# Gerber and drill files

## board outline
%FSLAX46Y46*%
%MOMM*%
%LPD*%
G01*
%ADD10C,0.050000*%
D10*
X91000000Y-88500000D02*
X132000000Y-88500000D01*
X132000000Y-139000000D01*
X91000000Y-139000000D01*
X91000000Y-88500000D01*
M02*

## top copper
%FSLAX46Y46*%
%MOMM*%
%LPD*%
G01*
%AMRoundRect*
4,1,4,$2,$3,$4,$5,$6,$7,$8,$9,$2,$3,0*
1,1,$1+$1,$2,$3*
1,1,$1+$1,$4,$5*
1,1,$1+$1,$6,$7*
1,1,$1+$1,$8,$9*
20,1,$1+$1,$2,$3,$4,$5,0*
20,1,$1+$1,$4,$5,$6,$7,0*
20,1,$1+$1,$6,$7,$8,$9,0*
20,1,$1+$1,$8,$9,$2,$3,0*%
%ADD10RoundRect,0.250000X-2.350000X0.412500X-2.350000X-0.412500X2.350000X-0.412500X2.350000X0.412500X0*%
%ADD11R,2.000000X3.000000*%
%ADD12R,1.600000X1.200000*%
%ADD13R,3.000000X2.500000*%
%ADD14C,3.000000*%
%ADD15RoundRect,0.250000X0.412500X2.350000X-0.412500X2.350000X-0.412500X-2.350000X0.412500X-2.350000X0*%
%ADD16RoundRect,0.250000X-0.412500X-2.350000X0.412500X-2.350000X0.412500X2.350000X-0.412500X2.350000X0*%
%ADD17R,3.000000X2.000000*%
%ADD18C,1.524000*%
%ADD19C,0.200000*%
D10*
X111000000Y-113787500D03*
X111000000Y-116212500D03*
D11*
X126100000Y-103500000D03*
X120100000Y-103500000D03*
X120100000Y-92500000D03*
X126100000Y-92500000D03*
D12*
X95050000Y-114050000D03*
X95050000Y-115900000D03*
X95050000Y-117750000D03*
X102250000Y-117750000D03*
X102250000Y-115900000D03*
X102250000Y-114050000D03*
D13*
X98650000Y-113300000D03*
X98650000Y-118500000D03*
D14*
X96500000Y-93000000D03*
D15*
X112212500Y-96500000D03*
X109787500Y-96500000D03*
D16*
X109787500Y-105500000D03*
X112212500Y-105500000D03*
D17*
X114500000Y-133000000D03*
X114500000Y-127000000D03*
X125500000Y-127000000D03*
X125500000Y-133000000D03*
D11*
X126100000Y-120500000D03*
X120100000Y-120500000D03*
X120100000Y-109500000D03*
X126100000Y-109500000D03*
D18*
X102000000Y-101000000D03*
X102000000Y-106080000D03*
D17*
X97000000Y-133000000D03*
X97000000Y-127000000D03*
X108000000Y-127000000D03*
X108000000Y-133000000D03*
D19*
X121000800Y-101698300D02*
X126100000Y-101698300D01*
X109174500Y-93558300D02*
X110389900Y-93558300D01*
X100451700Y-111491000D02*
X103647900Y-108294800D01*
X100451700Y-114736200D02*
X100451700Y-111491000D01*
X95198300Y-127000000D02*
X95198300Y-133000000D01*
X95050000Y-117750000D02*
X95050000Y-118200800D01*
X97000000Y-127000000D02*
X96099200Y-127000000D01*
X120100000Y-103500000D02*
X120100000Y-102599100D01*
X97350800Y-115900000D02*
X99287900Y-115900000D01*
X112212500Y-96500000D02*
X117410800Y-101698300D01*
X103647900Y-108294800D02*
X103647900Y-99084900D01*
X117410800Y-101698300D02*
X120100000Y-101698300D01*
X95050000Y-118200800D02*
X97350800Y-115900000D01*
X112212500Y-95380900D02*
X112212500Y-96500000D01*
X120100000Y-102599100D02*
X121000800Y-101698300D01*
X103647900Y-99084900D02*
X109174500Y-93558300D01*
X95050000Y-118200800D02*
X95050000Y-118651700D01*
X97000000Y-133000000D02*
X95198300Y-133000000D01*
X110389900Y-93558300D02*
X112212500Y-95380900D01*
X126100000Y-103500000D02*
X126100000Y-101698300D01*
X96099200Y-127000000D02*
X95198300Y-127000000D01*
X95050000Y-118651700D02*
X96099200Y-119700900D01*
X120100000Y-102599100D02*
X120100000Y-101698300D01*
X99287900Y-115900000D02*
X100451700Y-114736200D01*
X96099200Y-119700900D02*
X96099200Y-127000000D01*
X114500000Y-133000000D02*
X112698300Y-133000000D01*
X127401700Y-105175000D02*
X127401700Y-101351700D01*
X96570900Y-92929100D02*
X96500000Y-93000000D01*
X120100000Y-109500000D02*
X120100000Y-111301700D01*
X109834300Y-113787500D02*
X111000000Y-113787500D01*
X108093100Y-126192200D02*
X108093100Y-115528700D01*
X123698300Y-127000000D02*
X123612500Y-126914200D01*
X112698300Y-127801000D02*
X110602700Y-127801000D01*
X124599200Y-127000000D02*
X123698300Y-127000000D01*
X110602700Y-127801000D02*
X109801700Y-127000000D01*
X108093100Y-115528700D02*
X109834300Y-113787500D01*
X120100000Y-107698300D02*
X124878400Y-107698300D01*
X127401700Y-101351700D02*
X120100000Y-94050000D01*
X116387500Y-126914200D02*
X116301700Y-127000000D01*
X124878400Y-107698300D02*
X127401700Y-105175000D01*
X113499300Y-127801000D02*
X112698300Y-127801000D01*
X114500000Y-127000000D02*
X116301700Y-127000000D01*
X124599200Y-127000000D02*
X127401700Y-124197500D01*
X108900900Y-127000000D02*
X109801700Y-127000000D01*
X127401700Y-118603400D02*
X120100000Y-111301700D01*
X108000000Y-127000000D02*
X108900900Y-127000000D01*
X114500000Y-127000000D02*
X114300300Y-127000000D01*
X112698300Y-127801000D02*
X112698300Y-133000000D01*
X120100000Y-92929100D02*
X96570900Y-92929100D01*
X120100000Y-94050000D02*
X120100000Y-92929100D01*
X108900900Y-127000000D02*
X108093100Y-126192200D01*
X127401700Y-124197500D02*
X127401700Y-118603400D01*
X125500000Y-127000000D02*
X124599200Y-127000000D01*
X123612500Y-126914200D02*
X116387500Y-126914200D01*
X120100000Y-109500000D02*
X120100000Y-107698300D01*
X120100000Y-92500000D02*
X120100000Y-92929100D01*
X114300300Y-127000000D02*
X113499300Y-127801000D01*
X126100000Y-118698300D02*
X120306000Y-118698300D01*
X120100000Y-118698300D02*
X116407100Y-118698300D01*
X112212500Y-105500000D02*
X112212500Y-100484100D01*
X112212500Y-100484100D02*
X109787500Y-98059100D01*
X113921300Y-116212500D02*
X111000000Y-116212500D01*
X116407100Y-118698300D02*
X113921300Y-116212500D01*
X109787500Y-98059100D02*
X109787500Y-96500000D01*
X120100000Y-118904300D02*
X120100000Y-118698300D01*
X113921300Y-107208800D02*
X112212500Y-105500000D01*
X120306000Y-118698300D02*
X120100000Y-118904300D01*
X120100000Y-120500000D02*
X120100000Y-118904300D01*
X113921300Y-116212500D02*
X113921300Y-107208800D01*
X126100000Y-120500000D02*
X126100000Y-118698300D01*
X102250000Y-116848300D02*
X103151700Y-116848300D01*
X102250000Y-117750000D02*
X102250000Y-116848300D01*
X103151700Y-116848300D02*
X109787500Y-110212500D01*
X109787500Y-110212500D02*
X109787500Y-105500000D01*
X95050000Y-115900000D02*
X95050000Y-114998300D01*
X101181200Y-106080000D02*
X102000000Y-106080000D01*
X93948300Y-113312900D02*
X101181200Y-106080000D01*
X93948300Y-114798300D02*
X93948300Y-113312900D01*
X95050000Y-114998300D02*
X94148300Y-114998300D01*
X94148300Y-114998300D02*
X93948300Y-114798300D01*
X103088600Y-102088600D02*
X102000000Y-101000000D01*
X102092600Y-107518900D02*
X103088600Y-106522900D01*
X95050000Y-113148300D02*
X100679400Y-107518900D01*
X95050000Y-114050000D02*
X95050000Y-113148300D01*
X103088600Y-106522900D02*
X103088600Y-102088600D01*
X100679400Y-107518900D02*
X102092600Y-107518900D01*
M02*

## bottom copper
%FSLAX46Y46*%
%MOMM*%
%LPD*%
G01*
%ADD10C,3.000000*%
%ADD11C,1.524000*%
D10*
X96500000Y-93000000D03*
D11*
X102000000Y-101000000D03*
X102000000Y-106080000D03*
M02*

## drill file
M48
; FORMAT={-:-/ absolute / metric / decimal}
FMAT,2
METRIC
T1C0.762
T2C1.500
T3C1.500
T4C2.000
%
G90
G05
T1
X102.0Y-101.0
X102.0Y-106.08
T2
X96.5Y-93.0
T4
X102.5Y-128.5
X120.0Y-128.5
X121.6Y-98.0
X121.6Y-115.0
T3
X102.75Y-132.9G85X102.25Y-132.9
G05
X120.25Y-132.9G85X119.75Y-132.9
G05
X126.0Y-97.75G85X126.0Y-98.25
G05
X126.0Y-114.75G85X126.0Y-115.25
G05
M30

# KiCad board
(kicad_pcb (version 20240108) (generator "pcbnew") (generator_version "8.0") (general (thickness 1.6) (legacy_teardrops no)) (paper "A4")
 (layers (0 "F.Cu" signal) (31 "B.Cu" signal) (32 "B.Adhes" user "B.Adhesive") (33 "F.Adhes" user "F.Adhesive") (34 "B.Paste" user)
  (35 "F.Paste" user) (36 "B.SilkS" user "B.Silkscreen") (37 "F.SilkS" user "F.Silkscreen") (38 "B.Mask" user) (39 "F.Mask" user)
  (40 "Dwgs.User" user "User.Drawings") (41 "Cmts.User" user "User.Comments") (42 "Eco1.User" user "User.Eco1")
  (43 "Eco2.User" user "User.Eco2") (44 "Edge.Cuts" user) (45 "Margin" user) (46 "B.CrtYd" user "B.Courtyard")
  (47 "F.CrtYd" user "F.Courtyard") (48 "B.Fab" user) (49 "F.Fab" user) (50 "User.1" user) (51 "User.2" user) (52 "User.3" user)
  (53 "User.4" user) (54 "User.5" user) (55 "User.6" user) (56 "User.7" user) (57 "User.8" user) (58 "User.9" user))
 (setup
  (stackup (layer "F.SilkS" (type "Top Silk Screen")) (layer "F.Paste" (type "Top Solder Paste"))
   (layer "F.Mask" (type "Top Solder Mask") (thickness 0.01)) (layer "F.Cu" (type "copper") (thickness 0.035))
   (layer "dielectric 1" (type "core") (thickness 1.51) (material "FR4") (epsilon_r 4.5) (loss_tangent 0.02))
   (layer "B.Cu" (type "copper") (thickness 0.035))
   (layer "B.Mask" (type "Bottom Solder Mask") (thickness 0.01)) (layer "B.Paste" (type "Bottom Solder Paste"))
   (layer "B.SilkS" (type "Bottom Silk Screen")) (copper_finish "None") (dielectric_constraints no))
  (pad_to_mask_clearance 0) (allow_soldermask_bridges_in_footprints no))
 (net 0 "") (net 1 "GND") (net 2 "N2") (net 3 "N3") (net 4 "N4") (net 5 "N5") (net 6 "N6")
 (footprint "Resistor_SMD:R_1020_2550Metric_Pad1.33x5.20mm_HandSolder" (layer "F.Cu") (at 111 115 -90)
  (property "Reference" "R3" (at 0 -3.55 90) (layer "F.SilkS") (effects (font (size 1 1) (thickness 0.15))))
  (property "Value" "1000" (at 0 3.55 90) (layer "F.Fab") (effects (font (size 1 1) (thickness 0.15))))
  (pad "1" smd roundrect (at -1.2125 0 270) (size 1.325 5.2) (layers "F.Cu" "F.Paste" "F.Mask") (roundrect_rratio 0.188679) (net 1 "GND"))
  (pad "2" smd roundrect (at 1.2125 0 270) (size 1.325 5.2) (layers "F.Cu" "F.Paste" "F.Mask") (roundrect_rratio 0.188679) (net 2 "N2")))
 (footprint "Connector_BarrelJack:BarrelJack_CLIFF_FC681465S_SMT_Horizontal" (layer "F.Cu") (at 123.1 98 180)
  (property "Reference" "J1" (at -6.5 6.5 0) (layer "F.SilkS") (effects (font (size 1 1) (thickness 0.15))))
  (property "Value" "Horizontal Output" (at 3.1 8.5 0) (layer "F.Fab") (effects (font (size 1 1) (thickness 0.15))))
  (pad "" np_thru_hole oval (at -2.9 0 270) (size 2 1.5) (drill oval 2 1.5) (layers "*.Cu" "*.Mask"))
  (pad "" np_thru_hole circle (at 1.5 0 270) (size 2 2) (drill 2) (layers "*.Cu" "*.Mask"))
  (pad "1" smd rect (at -3 -5.5 270) (size 3 2) (layers "F.Cu" "F.Paste" "F.Mask") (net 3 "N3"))
  (pad "1" smd rect (at 3 -5.5 270) (size 3 2) (layers "F.Cu" "F.Paste" "F.Mask") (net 3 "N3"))
  (pad "2" smd rect (at 3 5.5 270) (size 3 2) (layers "F.Cu" "F.Paste" "F.Mask") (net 1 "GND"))
  (pad "3" smd rect (at -3 5.5 270) (size 3 2) (layers "F.Cu" "F.Paste" "F.Mask")))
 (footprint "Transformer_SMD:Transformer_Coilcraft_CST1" (layer "F.Cu") (at 98.65 115.9)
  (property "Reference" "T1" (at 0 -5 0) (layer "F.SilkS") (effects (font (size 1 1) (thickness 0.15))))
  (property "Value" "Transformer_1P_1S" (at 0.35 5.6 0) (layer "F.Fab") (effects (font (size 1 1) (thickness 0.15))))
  (pad "1" smd rect (at -3.6 -1.85) (size 1.6 1.2) (layers "F.Cu" "F.Paste" "F.Mask") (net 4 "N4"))
  (pad "2" smd rect (at -3.6 0) (size 1.6 1.2) (layers "F.Cu" "F.Paste" "F.Mask") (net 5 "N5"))
  (pad "3" smd rect (at -3.6 1.85) (size 1.6 1.2) (layers "F.Cu" "F.Paste" "F.Mask") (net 3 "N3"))
  (pad "4" smd rect (at 3.6 1.85) (size 1.6 1.2) (layers "F.Cu" "F.Paste" "F.Mask") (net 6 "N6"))
  (pad "5" smd rect (at 3.6 0) (size 1.6 1.2) (layers "F.Cu" "F.Paste" "F.Mask"))
  (pad "6" smd rect (at 3.6 -1.85) (size 1.6 1.2) (layers "F.Cu" "F.Paste" "F.Mask"))
  (pad "7" smd rect (at 0 -2.6) (size 3 2.5) (layers "F.Cu" "F.Paste" "F.Mask"))
  (pad "8" smd rect (at 0 2.6) (size 3 2.5) (layers "F.Cu" "F.Paste" "F.Mask")))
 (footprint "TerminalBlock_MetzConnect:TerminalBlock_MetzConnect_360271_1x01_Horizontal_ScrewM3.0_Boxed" (layer "F.Cu") (at 96.5 93)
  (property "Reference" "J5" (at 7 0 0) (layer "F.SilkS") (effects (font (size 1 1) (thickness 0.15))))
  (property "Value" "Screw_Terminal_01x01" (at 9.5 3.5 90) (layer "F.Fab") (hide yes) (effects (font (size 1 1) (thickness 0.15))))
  (pad "1" thru_hole circle (at 0 0) (size 3 3) (drill 1.5) (layers "*.Cu" "*.Mask") (remove_unused_layers no) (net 1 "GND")))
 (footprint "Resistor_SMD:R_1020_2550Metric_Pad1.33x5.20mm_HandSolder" (layer "F.Cu") (at 111 96.5 180)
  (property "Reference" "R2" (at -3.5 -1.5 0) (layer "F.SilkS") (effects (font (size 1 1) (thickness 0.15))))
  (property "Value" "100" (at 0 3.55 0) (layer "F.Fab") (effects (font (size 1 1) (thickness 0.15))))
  (pad "1" smd roundrect (at -1.2125 0 180) (size 1.325 5.2) (layers "F.Cu" "F.Paste" "F.Mask") (roundrect_rratio 0.188679) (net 3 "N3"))
  (pad "2" smd roundrect (at 1.2125 0 180) (size 1.325 5.2) (layers "F.Cu" "F.Paste" "F.Mask") (roundrect_rratio 0.188679) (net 2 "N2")))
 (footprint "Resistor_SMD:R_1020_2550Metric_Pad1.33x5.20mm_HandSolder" (layer "F.Cu") (at 111 105.5)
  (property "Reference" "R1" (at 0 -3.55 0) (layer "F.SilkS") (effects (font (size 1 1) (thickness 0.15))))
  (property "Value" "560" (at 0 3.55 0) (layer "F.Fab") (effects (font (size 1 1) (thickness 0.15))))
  (pad "1" smd roundrect (at -1.2125 0) (size 1.325 5.2) (layers "F.Cu" "F.Paste" "F.Mask") (roundrect_rratio 0.188679) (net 6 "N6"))
  (pad "2" smd roundrect (at 1.2125 0) (size 1.325 5.2) (layers "F.Cu" "F.Paste" "F.Mask") (roundrect_rratio 0.188679) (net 2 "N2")))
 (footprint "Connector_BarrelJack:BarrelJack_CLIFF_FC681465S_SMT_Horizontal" (layer "F.Cu") (at 120 130 90)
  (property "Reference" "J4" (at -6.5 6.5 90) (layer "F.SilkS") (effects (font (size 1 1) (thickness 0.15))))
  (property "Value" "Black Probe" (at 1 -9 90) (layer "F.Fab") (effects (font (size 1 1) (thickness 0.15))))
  (pad "" np_thru_hole oval (at -2.9 0 180) (size 2 1.5) (drill oval 2 1.5) (layers "*.Cu" "*.Mask"))
  (pad "" np_thru_hole circle (at 1.5 0 180) (size 2 2) (drill 2) (layers "*.Cu" "*.Mask"))
  (pad "1" smd rect (at -3 -5.5 180) (size 3 2) (layers "F.Cu" "F.Paste" "F.Mask") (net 1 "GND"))
  (pad "1" smd rect (at 3 -5.5 180) (size 3 2) (layers "F.Cu" "F.Paste" "F.Mask") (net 1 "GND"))
  (pad "2" smd rect (at 3 5.5 180) (size 3 2) (layers "F.Cu" "F.Paste" "F.Mask") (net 1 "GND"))
  (pad "3" smd rect (at -3 5.5 180) (size 3 2) (layers "F.Cu" "F.Paste" "F.Mask")))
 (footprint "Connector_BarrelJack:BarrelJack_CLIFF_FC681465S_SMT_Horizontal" (layer "F.Cu") (at 123.1 115 180)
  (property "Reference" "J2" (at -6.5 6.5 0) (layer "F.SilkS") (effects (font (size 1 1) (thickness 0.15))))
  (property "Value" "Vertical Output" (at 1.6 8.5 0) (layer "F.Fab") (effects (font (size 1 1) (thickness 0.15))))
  (pad "" np_thru_hole oval (at -2.9 0 270) (size 2 1.5) (drill oval 2 1.5) (layers "*.Cu" "*.Mask"))
  (pad "" np_thru_hole circle (at 1.5 0 270) (size 2 2) (drill 2) (layers "F&B.Cu" "*.Mask"))
  (pad "1" smd rect (at -3 -5.5 270) (size 3 2) (layers "F.Cu" "F.Paste" "F.Mask") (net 2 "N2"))
  (pad "1" smd rect (at 3 -5.5 270) (size 3 2) (layers "F.Cu" "F.Paste" "F.Mask") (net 2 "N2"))
  (pad "2" smd rect (at 3 5.5 270) (size 3 2) (layers "F.Cu" "F.Paste" "F.Mask") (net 1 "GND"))
  (pad "3" smd rect (at -3 5.5 270) (size 3 2) (layers "F.Cu" "F.Paste" "F.Mask")))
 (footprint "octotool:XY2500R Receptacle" (layer "F.Cu") (at 92 99.5 -90)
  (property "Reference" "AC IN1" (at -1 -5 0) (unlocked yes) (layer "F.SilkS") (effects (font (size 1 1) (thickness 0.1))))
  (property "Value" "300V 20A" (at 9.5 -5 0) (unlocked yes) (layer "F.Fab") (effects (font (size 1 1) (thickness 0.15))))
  (pad "1" thru_hole circle (at 1.5 -10 270) (size 1.524 1.524) (drill 0.762) (layers "*.Cu" "*.Mask") (remove_unused_layers no)
   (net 4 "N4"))
  (pad "2" thru_hole circle (at 6.58 -10 270) (size 1.524 1.524) (drill 0.762) (layers "*.Cu" "*.Mask") (remove_unused_layers no)
   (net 5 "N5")))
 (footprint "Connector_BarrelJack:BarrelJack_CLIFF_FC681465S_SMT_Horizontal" (layer "F.Cu") (at 102.5 130 90)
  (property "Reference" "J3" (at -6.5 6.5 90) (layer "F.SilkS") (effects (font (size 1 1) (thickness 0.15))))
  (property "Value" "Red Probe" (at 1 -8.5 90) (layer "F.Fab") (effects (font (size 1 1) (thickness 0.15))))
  (pad "" np_thru_hole oval (at -2.9 0 180) (size 2 1.5) (drill oval 2 1.5) (layers "*.Cu" "*.Mask"))
  (pad "" np_thru_hole circle (at 1.5 0 180) (size 2 2) (drill 2) (layers "*.Cu" "*.Mask"))
  (pad "1" smd rect (at -3 -5.5 180) (size 3 2) (layers "F.Cu" "F.Paste" "F.Mask") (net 3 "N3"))
  (pad "1" smd rect (at 3 -5.5 180) (size 3 2) (layers "F.Cu" "F.Paste" "F.Mask") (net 3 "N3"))
  (pad "2" smd rect (at 3 5.5 180) (size 3 2) (layers "F.Cu" "F.Paste" "F.Mask") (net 1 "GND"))
  (pad "3" smd rect (at -3 5.5 180) (size 3 2) (layers "F.Cu" "F.Paste" "F.Mask")))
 (gr_rect (start 91 88.5) (end 132 139) (locked yes) (stroke (width 0.05) (type default)) (fill none) (layer "Edge.Cuts"))
 (segment (start 121.0008 101.6983) (end 126.1 101.6983) (width 0.2) (layer "F.Cu") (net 3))
 (segment (start 109.1745 93.5583) (end 110.3899 93.5583) (width 0.2) (layer "F.Cu") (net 3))
 (segment (start 100.4517 111.491) (end 103.6479 108.2948) (width 0.2) (layer "F.Cu") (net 3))
 (segment (start 100.4517 114.7362) (end 100.4517 111.491) (width 0.2) (layer "F.Cu") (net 3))
 (segment (start 95.1983 127) (end 95.1983 133) (width 0.2) (layer "F.Cu") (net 3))
 (segment (start 95.05 117.75) (end 95.05 118.2008) (width 0.2) (layer "F.Cu") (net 3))
 (segment (start 97 127) (end 96.0992 127) (width 0.2) (layer "F.Cu") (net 3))
 (segment (start 120.1 103.5) (end 120.1 102.5991) (width 0.2) (layer "F.Cu") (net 3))
 (segment (start 97.3508 115.9) (end 99.2879 115.9) (width 0.2) (layer "F.Cu") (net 3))
 (segment (start 112.2125 96.5) (end 117.4108 101.6983) (width 0.2) (layer "F.Cu") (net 3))
 (segment (start 103.6479 108.2948) (end 103.6479 99.0849) (width 0.2) (layer "F.Cu") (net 3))
 (segment (start 117.4108 101.6983) (end 120.1 101.6983) (width 0.2) (layer "F.Cu") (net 3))
 (segment (start 95.05 118.2008) (end 97.3508 115.9) (width 0.2) (layer "F.Cu") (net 3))
 (segment (start 112.2125 95.3809) (end 112.2125 96.5) (width 0.2) (layer "F.Cu") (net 3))
 (segment (start 120.1 102.5991) (end 121.0008 101.6983) (width 0.2) (layer "F.Cu") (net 3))
 (segment (start 103.6479 99.0849) (end 109.1745 93.5583) (width 0.2) (layer "F.Cu") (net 3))
 (segment (start 95.05 118.2008) (end 95.05 118.6517) (width 0.2) (layer "F.Cu") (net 3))
 (segment (start 97 133) (end 95.1983 133) (width 0.2) (layer "F.Cu") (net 3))
 (segment (start 110.3899 93.5583) (end 112.2125 95.3809) (width 0.2) (layer "F.Cu") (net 3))
 (segment (start 126.1 103.5) (end 126.1 101.6983) (width 0.2) (layer "F.Cu") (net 3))
 (segment (start 96.0992 127) (end 95.1983 127) (width 0.2) (layer "F.Cu") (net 3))
 (segment (start 95.05 118.6517) (end 96.0992 119.7009) (width 0.2) (layer "F.Cu") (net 3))
 (segment (start 120.1 102.5991) (end 120.1 101.6983) (width 0.2) (layer "F.Cu") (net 3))
 (segment (start 99.2879 115.9) (end 100.4517 114.7362) (width 0.2) (layer "F.Cu") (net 3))
 (segment (start 96.0992 119.7009) (end 96.0992 127) (width 0.2) (layer "F.Cu") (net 3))
 (segment (start 114.5 133) (end 112.6983 133) (width 0.2) (layer "F.Cu") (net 1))
 (segment (start 127.4017 105.175) (end 127.4017 101.3517) (width 0.2) (layer "F.Cu") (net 1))
 (segment (start 96.5709 92.9291) (end 96.5 93) (width 0.2) (layer "F.Cu") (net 1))
 (segment (start 120.1 109.5) (end 120.1 111.3017) (width 0.2) (layer "F.Cu") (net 1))
 (segment (start 109.8343 113.7875) (end 111 113.7875) (width 0.2) (layer "F.Cu") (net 1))
 (segment (start 108.0931 126.1922) (end 108.0931 115.5287) (width 0.2) (layer "F.Cu") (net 1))
 (segment (start 123.6983 127) (end 123.6125 126.9142) (width 0.2) (layer "F.Cu") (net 1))
 (segment (start 112.6983 127.801) (end 110.6027 127.801) (width 0.2) (layer "F.Cu") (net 1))
 (segment (start 124.5992 127) (end 123.6983 127) (width 0.2) (layer "F.Cu") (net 1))
 (segment (start 110.6027 127.801) (end 109.8017 127) (width 0.2) (layer "F.Cu") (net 1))
 (segment (start 108.0931 115.5287) (end 109.8343 113.7875) (width 0.2) (layer "F.Cu") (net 1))
 (segment (start 120.1 107.6983) (end 124.8784 107.6983) (width 0.2) (layer "F.Cu") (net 1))
 (segment (start 127.4017 101.3517) (end 120.1 94.05) (width 0.2) (layer "F.Cu") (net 1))
 (segment (start 116.3875 126.9142) (end 116.3017 127) (width 0.2) (layer "F.Cu") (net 1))
 (segment (start 124.8784 107.6983) (end 127.4017 105.175) (width 0.2) (layer "F.Cu") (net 1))
 (segment (start 113.4993 127.801) (end 112.6983 127.801) (width 0.2) (layer "F.Cu") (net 1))
 (segment (start 114.5 127) (end 116.3017 127) (width 0.2) (layer "F.Cu") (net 1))
 (segment (start 124.5992 127) (end 127.4017 124.1975) (width 0.2) (layer "F.Cu") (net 1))
 (segment (start 108.9009 127) (end 109.8017 127) (width 0.2) (layer "F.Cu") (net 1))
 (segment (start 127.4017 118.6034) (end 120.1 111.3017) (width 0.2) (layer "F.Cu") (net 1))
 (segment (start 108 127) (end 108.9009 127) (width 0.2) (layer "F.Cu") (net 1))
 (segment (start 114.5 127) (end 114.3003 127) (width 0.2) (layer "F.Cu") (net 1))
 (segment (start 112.6983 127.801) (end 112.6983 133) (width 0.2) (layer "F.Cu") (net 1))
 (segment (start 120.1 92.9291) (end 96.5709 92.9291) (width 0.2) (layer "F.Cu") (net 1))
 (segment (start 120.1 94.05) (end 120.1 92.9291) (width 0.2) (layer "F.Cu") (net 1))
 (segment (start 108.9009 127) (end 108.0931 126.1922) (width 0.2) (layer "F.Cu") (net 1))
 (segment (start 127.4017 124.1975) (end 127.4017 118.6034) (width 0.2) (layer "F.Cu") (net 1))
 (segment (start 125.5 127) (end 124.5992 127) (width 0.2) (layer "F.Cu") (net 1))
 (segment (start 123.6125 126.9142) (end 116.3875 126.9142) (width 0.2) (layer "F.Cu") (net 1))
 (segment (start 120.1 109.5) (end 120.1 107.6983) (width 0.2) (layer "F.Cu") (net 1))
 (segment (start 120.1 92.5) (end 120.1 92.9291) (width 0.2) (layer "F.Cu") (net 1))
 (segment (start 114.3003 127) (end 113.4993 127.801) (width 0.2) (layer "F.Cu") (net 1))
 (segment (start 126.1 118.6983) (end 120.306 118.6983) (width 0.2) (layer "F.Cu") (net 2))
 (segment (start 120.1 118.6983) (end 116.4071 118.6983) (width 0.2) (layer "F.Cu") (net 2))
 (segment (start 112.2125 105.5) (end 112.2125 100.4841) (width 0.2) (layer "F.Cu") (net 2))
 (segment (start 112.2125 100.4841) (end 109.7875 98.0591) (width 0.2) (layer "F.Cu") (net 2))
 (segment (start 113.9213 116.2125) (end 111 116.2125) (width 0.2) (layer "F.Cu") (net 2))
 (segment (start 116.4071 118.6983) (end 113.9213 116.2125) (width 0.2) (layer "F.Cu") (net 2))
 (segment (start 109.7875 98.0591) (end 109.7875 96.5) (width 0.2) (layer "F.Cu") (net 2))
 (segment (start 120.1 118.9043) (end 120.1 118.6983) (width 0.2) (layer "F.Cu") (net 2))
 (segment (start 113.9213 107.2088) (end 112.2125 105.5) (width 0.2) (layer "F.Cu") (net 2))
 (segment (start 120.306 118.6983) (end 120.1 118.9043) (width 0.2) (layer "F.Cu") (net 2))
 (segment (start 120.1 120.5) (end 120.1 118.9043) (width 0.2) (layer "F.Cu") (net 2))
 (segment (start 113.9213 116.2125) (end 113.9213 107.2088) (width 0.2) (layer "F.Cu") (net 2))
 (segment (start 126.1 120.5) (end 126.1 118.6983) (width 0.2) (layer "F.Cu") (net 2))
 (segment (start 102.25 116.8483) (end 103.1517 116.8483) (width 0.2) (layer "F.Cu") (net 6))
 (segment (start 102.25 117.75) (end 102.25 116.8483) (width 0.2) (layer "F.Cu") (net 6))
 (segment (start 103.1517 116.8483) (end 109.7875 110.2125) (width 0.2) (layer "F.Cu") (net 6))
 (segment (start 109.7875 110.2125) (end 109.7875 105.5) (width 0.2) (layer "F.Cu") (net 6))
 (segment (start 95.05 115.9) (end 95.05 114.9983) (width 0.2) (layer "F.Cu") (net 5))
 (segment (start 101.1812 106.08) (end 102 106.08) (width 0.2) (layer "F.Cu") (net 5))
 (segment (start 93.9483 113.3129) (end 101.1812 106.08) (width 0.2) (layer "F.Cu") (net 5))
 (segment (start 93.9483 114.7983) (end 93.9483 113.3129) (width 0.2) (layer "F.Cu") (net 5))
 (segment (start 95.05 114.9983) (end 94.1483 114.9983) (width 0.2) (layer "F.Cu") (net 5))
 (segment (start 94.1483 114.9983) (end 93.9483 114.7983) (width 0.2) (layer "F.Cu") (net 5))
 (segment (start 103.0886 102.0886) (end 102 101) (width 0.2) (layer "F.Cu") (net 4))
 (segment (start 102.0926 107.5189) (end 103.0886 106.5229) (width 0.2) (layer "F.Cu") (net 4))
 (segment (start 95.05 113.1483) (end 100.6794 107.5189) (width 0.2) (layer "F.Cu") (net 4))
 (segment (start 95.05 114.05) (end 95.05 113.1483) (width 0.2) (layer "F.Cu") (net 4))
 (segment (start 103.0886 106.5229) (end 103.0886 102.0886) (width 0.2) (layer "F.Cu") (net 4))
 (segment (start 100.6794 107.5189) (end 102.0926 107.5189) (width 0.2) (layer "F.Cu") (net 4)))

